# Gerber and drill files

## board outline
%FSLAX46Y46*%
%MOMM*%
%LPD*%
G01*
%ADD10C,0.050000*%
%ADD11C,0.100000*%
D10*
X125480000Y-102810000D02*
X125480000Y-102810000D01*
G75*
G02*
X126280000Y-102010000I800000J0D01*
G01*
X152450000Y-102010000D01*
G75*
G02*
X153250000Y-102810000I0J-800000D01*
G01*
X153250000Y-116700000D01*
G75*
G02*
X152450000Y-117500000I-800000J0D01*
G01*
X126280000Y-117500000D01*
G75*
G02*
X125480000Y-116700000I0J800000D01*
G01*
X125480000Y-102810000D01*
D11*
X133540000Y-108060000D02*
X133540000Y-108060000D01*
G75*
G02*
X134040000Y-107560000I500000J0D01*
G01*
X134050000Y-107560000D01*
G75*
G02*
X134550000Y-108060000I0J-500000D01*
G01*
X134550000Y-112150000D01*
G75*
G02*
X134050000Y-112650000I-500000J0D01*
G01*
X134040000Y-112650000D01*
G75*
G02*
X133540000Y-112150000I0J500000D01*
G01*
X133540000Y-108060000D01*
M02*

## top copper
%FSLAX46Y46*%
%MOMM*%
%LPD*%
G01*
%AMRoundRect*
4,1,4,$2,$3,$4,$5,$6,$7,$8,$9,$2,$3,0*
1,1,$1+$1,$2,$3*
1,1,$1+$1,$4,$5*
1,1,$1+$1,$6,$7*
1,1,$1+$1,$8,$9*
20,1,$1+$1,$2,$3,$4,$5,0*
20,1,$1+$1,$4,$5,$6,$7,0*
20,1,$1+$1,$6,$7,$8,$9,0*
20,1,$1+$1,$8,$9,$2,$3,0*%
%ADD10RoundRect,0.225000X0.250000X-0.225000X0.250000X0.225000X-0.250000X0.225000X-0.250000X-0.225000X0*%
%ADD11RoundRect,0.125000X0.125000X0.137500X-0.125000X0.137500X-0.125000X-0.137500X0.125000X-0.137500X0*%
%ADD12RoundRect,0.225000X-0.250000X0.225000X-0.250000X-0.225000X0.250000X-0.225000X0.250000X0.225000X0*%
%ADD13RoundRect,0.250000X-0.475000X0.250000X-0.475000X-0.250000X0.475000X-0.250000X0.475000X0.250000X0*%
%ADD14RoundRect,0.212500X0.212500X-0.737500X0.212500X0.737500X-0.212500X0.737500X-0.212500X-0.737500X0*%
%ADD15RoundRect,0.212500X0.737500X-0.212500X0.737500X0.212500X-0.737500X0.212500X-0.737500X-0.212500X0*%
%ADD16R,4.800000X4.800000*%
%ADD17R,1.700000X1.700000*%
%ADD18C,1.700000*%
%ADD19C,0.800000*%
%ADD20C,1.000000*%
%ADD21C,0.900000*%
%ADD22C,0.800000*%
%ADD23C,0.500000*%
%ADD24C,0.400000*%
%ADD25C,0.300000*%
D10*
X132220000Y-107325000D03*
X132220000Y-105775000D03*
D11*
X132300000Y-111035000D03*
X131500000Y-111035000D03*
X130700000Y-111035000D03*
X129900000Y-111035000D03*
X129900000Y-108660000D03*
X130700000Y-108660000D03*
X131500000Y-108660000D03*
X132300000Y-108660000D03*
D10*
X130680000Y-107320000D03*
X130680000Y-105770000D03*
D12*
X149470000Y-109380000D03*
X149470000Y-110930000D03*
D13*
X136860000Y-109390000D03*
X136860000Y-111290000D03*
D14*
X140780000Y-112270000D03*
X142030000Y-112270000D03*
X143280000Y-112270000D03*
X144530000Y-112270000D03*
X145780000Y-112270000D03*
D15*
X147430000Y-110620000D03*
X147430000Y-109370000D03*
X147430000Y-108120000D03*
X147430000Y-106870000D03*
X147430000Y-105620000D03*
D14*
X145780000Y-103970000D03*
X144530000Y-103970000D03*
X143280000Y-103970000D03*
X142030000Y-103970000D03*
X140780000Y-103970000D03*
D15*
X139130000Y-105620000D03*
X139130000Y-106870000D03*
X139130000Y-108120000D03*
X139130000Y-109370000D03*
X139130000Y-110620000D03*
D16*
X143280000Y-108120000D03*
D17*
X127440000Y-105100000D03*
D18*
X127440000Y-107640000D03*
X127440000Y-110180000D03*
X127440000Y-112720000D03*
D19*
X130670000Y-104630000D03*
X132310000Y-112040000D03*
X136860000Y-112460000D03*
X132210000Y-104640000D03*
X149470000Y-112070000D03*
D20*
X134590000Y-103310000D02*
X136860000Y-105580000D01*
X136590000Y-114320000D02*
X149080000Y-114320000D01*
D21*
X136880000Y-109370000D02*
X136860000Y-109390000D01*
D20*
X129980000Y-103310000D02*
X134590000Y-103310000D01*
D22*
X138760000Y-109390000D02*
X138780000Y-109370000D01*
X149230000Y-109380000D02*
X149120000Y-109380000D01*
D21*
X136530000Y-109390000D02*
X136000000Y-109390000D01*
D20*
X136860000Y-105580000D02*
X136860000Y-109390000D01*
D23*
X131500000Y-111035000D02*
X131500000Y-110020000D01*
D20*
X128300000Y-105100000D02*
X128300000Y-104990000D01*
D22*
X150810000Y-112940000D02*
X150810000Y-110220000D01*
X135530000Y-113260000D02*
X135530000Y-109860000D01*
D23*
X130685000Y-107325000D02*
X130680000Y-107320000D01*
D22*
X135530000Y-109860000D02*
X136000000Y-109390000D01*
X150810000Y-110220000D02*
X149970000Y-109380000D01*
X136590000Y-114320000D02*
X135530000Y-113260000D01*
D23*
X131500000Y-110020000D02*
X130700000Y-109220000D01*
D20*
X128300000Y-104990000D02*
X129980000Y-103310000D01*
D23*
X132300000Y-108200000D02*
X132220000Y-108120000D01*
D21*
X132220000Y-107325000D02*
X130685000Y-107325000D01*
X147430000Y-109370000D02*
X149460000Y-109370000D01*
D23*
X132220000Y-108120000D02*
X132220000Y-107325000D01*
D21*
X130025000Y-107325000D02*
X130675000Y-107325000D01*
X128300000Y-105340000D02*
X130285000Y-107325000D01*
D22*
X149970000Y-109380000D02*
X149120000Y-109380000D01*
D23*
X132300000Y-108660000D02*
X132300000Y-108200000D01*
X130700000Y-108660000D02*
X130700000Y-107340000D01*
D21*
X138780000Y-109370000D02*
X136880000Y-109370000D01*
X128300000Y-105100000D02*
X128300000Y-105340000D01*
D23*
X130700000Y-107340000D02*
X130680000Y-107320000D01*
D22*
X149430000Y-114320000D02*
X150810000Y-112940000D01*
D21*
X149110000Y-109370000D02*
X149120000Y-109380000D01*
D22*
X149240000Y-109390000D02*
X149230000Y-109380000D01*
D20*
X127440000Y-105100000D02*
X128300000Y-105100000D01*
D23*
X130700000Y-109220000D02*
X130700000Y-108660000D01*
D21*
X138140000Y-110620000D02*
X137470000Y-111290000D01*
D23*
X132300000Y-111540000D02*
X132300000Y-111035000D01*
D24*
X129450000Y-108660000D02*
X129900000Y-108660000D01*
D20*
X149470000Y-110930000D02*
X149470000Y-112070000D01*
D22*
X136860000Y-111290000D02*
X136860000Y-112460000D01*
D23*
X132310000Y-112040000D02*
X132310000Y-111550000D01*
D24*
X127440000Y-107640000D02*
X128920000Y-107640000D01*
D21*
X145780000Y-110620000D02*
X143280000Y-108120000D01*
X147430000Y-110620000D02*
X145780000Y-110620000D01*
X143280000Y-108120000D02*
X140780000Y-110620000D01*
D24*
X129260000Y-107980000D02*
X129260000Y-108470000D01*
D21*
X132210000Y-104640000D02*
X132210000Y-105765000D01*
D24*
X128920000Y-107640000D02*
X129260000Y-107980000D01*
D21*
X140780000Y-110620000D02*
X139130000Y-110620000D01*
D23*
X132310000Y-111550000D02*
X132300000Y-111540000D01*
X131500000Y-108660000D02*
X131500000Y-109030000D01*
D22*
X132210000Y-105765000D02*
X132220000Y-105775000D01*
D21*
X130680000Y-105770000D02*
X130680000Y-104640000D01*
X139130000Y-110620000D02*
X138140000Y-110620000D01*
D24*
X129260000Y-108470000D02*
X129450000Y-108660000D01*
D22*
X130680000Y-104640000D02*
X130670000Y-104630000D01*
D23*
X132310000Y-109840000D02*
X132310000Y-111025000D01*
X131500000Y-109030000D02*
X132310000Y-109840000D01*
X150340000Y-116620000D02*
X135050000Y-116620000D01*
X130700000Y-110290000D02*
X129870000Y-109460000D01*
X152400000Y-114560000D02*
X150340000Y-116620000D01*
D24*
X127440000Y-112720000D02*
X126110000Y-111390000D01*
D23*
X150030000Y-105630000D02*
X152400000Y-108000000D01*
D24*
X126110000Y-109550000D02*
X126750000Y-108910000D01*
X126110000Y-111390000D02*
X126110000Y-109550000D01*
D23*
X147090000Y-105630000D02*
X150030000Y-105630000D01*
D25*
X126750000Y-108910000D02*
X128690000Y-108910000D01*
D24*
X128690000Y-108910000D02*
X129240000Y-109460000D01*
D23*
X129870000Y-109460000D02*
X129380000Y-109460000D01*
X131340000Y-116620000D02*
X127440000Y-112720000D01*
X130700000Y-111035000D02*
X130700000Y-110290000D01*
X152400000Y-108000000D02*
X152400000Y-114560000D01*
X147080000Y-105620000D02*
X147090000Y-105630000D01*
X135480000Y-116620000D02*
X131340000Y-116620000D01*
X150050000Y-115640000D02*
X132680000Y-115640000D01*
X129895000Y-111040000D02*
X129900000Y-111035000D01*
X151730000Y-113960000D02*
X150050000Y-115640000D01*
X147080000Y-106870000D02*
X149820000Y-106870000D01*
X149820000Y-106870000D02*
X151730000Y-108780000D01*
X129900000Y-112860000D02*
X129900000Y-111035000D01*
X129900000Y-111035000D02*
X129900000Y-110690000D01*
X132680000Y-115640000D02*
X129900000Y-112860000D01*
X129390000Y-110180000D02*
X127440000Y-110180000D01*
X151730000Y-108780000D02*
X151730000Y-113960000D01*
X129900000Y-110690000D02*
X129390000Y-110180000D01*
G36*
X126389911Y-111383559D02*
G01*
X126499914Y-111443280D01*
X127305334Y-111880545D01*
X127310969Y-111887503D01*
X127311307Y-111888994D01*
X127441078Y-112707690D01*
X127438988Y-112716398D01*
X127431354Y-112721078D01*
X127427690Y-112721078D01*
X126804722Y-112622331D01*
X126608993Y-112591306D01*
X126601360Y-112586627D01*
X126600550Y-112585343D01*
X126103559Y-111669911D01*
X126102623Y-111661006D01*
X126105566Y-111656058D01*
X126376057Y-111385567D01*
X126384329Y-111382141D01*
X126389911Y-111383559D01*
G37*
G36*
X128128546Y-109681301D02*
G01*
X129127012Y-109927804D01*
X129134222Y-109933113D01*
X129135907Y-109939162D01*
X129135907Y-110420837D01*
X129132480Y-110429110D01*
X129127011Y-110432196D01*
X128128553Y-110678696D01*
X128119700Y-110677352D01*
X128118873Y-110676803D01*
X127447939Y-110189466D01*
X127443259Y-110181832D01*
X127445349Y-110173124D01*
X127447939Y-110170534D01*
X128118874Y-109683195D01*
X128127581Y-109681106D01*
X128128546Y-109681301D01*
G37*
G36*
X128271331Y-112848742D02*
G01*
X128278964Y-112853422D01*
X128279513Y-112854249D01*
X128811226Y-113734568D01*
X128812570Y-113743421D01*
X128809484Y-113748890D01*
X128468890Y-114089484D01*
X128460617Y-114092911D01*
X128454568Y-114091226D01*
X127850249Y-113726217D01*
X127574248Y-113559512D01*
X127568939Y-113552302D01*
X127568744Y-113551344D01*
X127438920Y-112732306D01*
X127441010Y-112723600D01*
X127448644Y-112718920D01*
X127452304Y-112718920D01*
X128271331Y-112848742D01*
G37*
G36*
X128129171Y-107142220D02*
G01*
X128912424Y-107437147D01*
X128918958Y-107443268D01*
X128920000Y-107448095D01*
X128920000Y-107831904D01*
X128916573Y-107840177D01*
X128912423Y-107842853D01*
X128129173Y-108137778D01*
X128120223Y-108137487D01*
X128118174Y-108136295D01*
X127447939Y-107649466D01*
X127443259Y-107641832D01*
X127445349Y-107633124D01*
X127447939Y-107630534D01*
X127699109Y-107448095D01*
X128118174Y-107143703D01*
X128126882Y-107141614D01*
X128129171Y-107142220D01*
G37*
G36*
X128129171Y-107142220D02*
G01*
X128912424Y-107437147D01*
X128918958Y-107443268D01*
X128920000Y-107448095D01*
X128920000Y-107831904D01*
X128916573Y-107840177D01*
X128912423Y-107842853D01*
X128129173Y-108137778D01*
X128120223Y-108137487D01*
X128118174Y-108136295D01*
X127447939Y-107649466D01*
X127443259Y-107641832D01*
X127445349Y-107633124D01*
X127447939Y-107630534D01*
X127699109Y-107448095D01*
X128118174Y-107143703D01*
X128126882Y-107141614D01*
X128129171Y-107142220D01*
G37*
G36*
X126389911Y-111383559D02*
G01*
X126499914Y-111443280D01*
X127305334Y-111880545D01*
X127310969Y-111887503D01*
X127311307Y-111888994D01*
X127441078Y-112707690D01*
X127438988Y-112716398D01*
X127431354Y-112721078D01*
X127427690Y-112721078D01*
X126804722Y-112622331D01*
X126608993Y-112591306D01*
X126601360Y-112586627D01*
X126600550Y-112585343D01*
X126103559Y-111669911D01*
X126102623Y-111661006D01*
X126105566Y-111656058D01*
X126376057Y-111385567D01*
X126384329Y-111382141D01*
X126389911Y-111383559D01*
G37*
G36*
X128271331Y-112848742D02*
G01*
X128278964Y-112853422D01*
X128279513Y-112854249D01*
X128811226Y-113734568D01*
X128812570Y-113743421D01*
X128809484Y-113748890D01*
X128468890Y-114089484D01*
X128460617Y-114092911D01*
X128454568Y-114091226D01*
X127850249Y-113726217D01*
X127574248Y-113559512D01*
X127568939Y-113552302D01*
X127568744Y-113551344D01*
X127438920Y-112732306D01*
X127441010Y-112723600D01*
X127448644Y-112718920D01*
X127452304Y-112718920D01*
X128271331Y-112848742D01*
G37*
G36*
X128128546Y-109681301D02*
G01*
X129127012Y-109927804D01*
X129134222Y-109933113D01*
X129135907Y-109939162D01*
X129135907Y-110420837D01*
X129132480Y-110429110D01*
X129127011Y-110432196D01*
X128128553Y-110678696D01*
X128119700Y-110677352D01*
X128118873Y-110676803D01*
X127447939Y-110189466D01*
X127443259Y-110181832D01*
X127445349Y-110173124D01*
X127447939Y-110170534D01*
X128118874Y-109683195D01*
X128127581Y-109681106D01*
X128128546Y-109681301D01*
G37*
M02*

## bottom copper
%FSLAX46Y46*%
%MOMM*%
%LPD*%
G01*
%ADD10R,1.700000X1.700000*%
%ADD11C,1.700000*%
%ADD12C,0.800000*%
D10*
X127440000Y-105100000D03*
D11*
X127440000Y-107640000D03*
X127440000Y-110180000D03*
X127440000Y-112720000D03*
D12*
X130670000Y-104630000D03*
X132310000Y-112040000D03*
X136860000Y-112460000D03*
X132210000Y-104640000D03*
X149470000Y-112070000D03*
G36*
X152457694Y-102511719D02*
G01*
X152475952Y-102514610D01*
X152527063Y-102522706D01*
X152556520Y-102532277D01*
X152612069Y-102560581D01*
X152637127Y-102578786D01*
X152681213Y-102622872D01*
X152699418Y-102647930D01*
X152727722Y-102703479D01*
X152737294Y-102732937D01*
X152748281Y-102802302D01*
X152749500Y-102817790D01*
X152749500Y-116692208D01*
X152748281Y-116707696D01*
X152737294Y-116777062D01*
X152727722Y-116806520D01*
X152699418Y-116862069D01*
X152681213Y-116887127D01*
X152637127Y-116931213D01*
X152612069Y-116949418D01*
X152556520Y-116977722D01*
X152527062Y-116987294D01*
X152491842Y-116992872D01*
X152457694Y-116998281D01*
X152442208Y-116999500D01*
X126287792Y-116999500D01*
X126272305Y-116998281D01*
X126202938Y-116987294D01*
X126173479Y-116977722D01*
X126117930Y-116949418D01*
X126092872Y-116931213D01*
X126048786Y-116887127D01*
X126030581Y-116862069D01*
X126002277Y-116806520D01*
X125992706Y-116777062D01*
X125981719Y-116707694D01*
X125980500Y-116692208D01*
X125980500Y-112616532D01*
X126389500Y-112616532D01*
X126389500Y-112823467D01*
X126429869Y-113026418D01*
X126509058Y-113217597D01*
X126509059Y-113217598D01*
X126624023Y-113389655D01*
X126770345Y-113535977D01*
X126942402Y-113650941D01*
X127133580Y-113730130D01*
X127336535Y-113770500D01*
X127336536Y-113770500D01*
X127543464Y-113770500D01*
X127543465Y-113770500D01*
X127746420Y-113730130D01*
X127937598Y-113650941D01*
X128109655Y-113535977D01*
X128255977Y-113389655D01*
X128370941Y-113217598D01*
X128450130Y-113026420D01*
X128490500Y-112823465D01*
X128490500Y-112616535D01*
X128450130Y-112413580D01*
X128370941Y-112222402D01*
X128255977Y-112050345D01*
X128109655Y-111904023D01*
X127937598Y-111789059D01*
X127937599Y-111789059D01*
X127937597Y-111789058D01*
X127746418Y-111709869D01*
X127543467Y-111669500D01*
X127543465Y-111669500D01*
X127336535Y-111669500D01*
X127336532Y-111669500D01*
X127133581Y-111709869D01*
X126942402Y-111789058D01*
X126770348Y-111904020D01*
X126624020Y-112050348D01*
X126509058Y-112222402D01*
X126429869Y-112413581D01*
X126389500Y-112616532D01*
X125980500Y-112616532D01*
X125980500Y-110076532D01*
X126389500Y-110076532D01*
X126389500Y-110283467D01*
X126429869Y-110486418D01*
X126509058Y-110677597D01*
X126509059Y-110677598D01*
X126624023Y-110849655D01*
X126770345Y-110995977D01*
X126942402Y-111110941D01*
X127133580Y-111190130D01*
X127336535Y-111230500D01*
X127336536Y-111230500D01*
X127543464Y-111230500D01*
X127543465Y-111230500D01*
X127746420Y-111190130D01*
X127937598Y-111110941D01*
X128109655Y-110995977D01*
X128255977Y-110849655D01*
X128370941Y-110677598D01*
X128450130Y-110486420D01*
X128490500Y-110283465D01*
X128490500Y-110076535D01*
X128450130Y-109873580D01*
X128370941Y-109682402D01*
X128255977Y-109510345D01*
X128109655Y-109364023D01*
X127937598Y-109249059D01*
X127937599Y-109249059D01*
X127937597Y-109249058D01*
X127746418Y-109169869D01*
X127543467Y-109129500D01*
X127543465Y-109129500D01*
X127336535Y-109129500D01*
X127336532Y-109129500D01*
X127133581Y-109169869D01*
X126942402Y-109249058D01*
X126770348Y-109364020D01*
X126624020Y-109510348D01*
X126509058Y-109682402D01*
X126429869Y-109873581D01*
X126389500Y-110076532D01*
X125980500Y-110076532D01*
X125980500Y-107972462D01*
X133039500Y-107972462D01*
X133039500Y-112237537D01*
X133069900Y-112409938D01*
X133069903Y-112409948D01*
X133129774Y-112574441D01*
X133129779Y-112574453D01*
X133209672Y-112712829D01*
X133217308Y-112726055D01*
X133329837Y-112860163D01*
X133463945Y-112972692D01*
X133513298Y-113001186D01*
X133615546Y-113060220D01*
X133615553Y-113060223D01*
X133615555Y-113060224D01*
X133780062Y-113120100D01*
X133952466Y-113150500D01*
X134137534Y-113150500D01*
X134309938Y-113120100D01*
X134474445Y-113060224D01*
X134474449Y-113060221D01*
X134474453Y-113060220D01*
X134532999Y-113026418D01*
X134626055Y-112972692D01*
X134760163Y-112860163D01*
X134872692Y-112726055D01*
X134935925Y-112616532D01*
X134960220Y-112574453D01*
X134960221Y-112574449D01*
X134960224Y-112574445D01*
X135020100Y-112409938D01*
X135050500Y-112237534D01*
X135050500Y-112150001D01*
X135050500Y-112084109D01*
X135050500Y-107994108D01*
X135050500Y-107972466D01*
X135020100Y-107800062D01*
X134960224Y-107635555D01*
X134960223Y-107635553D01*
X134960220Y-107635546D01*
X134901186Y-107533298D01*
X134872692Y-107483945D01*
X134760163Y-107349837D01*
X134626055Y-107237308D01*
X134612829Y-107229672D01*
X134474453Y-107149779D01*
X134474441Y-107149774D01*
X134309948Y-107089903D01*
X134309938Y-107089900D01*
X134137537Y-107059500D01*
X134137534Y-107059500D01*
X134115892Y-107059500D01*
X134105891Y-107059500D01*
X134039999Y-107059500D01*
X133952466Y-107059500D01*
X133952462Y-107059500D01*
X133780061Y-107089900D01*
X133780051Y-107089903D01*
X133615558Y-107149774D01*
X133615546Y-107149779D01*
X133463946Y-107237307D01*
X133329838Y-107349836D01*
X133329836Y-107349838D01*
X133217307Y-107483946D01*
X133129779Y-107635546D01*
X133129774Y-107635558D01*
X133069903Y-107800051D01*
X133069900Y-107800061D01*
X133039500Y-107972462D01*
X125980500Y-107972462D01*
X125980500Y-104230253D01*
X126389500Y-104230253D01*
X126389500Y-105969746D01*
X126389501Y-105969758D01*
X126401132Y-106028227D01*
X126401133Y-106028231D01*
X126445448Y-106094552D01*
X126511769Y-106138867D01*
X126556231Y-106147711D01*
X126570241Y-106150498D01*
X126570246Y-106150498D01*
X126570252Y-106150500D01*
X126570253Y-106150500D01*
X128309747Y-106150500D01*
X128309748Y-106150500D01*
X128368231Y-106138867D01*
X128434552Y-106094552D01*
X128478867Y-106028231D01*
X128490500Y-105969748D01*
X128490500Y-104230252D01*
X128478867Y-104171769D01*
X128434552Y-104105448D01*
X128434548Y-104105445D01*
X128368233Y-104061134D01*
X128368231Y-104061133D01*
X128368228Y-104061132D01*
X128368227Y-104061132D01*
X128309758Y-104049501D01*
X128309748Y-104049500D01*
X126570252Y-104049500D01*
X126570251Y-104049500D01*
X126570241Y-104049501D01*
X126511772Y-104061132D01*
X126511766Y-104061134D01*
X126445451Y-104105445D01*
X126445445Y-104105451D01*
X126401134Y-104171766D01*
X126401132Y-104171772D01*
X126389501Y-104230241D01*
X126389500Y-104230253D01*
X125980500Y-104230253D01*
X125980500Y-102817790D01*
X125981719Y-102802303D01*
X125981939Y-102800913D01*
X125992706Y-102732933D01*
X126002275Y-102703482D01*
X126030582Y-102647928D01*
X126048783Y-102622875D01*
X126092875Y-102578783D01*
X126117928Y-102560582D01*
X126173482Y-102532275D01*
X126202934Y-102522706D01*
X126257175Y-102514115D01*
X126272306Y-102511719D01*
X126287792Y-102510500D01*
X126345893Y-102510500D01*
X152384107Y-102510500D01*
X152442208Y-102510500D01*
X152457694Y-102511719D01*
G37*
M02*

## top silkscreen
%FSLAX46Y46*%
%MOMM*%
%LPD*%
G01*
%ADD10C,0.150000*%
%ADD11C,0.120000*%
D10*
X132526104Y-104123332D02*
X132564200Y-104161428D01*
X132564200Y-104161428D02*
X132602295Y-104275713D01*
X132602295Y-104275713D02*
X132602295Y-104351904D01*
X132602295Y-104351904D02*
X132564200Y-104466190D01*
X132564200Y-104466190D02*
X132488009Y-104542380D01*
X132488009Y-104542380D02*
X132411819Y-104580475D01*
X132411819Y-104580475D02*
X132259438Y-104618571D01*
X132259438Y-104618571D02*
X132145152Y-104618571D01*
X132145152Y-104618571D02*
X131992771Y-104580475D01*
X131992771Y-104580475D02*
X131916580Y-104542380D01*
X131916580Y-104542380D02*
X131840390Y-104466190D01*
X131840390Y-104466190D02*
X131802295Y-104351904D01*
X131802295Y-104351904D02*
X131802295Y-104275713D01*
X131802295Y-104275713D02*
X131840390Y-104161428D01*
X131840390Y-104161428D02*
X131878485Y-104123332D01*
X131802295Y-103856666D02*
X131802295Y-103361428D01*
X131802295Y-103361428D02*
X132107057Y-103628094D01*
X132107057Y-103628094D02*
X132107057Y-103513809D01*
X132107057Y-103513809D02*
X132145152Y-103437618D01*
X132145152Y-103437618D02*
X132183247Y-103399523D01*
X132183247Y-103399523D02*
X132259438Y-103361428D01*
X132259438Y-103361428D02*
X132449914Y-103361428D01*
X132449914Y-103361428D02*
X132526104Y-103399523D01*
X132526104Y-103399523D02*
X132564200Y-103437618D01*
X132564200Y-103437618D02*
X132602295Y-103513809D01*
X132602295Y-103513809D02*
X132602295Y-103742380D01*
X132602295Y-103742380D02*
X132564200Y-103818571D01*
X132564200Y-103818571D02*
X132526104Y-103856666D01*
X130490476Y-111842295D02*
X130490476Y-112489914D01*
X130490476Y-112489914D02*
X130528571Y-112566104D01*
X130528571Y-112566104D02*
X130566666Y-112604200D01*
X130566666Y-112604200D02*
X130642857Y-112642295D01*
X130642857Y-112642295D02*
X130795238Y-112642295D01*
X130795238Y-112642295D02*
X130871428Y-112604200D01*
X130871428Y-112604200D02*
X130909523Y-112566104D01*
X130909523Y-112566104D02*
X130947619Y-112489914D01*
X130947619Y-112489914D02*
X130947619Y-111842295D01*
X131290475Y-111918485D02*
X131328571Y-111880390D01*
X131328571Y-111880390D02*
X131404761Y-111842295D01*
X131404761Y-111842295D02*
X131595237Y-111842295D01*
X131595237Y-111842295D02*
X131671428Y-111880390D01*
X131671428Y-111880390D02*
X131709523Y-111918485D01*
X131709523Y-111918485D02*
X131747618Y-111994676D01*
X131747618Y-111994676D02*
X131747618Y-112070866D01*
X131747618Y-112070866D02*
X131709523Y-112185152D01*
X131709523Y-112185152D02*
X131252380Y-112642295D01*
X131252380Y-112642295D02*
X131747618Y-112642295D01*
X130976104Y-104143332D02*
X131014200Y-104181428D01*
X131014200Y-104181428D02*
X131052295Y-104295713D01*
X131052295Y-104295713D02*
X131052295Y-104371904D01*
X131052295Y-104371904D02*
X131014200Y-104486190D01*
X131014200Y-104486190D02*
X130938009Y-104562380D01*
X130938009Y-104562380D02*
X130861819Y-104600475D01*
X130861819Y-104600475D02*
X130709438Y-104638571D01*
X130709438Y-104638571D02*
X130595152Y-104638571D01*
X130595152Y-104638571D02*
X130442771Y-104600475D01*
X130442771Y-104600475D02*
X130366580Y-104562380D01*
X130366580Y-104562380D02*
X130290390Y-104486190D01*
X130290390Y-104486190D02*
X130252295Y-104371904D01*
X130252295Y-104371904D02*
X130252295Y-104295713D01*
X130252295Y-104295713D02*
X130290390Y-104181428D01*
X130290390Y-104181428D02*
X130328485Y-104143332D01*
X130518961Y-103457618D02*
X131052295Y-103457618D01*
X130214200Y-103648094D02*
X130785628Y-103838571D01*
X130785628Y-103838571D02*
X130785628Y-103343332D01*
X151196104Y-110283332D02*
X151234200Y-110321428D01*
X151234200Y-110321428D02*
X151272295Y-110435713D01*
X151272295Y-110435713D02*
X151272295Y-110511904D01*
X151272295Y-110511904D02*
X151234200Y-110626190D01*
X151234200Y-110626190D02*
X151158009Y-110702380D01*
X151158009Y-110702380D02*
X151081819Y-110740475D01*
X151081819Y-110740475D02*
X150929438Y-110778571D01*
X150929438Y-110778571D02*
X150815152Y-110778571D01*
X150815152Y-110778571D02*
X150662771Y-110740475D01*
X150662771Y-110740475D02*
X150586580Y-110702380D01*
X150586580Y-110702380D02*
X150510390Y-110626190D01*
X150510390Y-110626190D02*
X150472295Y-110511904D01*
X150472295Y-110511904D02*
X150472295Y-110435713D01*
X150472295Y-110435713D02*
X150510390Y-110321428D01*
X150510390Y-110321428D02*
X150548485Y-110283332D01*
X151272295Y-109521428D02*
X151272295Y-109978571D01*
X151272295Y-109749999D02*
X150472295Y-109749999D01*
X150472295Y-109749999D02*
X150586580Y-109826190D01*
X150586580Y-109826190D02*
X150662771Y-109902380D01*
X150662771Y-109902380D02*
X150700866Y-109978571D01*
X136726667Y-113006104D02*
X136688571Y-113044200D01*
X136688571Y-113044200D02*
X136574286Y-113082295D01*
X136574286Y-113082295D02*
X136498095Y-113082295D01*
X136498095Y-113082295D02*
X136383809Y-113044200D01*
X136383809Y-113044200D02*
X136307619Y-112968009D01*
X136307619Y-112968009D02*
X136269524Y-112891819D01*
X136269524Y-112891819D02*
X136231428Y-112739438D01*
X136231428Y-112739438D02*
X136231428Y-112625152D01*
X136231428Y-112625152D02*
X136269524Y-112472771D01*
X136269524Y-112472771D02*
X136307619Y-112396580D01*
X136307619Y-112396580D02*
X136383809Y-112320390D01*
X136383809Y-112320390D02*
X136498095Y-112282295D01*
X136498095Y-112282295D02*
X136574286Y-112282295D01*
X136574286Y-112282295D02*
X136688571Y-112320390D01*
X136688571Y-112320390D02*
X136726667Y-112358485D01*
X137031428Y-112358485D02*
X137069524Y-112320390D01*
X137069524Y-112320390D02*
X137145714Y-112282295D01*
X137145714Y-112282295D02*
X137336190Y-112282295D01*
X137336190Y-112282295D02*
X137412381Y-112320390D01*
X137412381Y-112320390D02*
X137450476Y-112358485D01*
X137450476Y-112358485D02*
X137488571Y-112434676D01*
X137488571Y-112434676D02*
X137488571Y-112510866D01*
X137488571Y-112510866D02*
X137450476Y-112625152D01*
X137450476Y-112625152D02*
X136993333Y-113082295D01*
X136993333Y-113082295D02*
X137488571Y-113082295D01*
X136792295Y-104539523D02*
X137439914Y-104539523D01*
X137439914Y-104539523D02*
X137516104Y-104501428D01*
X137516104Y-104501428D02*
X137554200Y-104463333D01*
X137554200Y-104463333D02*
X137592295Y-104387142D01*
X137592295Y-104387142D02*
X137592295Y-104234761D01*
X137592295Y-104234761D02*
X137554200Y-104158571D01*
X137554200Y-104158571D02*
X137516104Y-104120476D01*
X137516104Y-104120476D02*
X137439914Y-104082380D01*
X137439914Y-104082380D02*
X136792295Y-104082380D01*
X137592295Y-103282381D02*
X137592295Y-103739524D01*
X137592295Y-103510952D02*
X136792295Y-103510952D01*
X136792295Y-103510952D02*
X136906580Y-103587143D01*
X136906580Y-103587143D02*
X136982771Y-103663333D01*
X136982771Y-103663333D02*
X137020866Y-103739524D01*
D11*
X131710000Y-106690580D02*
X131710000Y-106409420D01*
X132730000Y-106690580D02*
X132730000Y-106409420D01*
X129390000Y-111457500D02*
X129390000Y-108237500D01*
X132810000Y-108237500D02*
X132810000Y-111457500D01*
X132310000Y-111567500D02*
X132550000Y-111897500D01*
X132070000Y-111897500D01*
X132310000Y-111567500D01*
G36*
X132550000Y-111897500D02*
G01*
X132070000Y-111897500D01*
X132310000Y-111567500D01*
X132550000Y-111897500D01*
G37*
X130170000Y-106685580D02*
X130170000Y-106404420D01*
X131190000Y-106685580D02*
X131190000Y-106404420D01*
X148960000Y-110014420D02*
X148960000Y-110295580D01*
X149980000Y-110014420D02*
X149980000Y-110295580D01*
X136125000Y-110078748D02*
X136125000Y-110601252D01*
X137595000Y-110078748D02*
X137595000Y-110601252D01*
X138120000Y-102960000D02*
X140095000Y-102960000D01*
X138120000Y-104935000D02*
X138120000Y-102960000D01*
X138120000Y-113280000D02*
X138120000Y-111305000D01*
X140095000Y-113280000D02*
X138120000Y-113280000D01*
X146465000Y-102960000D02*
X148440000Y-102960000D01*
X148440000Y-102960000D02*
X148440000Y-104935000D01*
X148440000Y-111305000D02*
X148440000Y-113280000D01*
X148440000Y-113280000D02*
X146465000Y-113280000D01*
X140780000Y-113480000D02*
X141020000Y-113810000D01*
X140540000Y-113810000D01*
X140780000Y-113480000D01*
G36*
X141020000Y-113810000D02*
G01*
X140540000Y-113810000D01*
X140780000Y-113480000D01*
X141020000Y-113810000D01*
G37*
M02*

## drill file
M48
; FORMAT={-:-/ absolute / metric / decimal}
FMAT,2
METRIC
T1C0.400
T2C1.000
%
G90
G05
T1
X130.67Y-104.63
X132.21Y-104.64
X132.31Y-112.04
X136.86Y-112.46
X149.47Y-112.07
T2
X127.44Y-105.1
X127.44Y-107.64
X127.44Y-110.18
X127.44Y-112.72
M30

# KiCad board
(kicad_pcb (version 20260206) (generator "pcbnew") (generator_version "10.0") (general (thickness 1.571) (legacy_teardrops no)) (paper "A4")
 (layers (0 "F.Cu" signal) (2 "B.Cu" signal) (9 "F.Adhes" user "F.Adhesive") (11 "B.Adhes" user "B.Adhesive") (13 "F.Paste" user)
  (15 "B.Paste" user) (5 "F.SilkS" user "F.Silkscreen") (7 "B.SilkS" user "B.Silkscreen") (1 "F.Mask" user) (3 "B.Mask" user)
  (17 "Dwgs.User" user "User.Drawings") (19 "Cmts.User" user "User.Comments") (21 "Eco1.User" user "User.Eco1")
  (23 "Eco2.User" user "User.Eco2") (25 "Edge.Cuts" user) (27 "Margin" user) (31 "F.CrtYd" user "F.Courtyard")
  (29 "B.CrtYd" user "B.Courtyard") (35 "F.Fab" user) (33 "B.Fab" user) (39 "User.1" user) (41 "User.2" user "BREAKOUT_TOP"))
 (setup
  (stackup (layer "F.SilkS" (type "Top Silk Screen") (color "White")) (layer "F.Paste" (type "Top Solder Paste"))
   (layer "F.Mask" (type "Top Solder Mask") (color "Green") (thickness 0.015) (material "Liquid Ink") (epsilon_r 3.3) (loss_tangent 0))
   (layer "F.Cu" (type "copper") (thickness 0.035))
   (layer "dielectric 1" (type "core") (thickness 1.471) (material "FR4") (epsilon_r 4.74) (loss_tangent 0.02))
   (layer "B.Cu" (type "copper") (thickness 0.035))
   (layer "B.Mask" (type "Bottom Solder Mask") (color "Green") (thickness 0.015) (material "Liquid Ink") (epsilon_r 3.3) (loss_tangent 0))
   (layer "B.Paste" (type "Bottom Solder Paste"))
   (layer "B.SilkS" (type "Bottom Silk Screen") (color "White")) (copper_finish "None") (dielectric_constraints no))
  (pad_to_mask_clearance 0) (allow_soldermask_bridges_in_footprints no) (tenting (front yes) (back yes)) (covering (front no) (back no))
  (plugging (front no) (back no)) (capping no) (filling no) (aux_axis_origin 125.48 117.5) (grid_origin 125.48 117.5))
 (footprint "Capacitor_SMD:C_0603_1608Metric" (layer "F.Cu") (at 132.22 106.55 90)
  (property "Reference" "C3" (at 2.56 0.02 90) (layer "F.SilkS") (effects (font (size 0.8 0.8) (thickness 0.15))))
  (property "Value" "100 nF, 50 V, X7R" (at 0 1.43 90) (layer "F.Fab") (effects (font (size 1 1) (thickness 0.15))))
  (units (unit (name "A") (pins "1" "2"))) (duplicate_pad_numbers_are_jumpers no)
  (fp_line (start -0.14058 -0.51) (end 0.14058 -0.51) (stroke (width 0.12) (type solid)) (layer "F.SilkS"))
  (fp_line (start -0.14058 0.51) (end 0.14058 0.51) (stroke (width 0.12) (type solid)) (layer "F.SilkS"))
  (pad "1" smd roundrect (at -0.775 0 90) (size 0.9 0.95) (layers "F.Cu" "F.Mask" "F.Paste") (roundrect_rratio 0.25) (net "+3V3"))
  (pad "2" smd roundrect (at 0.775 0 90) (size 0.9 0.95) (layers "F.Cu" "F.Mask" "F.Paste") (roundrect_rratio 0.25) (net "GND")))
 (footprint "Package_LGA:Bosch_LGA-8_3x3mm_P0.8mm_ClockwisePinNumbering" (layer "F.Cu") (at 131.1 109.8475 180)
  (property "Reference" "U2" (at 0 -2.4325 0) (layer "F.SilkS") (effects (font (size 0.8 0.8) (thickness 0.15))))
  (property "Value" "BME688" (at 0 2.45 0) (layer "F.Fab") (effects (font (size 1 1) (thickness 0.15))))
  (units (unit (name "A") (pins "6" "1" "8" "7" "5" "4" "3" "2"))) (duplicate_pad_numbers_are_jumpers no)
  (fp_line (start 1.71 -1.61) (end 1.71 1.61) (stroke (width 0.12) (type solid)) (layer "F.SilkS"))
  (fp_line (start -1.71 1.61) (end -1.71 -1.61) (stroke (width 0.12) (type solid)) (layer "F.SilkS"))
  (fp_poly (pts (xy -1.21 -1.72) (xy -1.45 -2.05) (xy -0.97 -2.05)) (stroke (width 0.12) (type solid)) (fill yes) (layer "F.SilkS"))
  (pad "1" smd roundrect (at -1.2 -1.1875 180) (size 0.5 0.525) (layers "F.Cu" "F.Mask" "F.Paste") (roundrect_rratio 0.25) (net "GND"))
  (pad "2" smd roundrect (at -0.4 -1.1875 180) (size 0.5 0.525) (layers "F.Cu" "F.Mask" "F.Paste") (roundrect_rratio 0.25) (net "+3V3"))
  (pad "3" smd roundrect (at 0.4 -1.1875 180) (size 0.5 0.525) (layers "F.Cu" "F.Mask" "F.Paste") (roundrect_rratio 0.25) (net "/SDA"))
  (pad "4" smd roundrect (at 1.2 -1.1875 180) (size 0.5 0.525) (layers "F.Cu" "F.Mask" "F.Paste") (roundrect_rratio 0.25) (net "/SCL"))
  (pad "5" smd roundrect (at 1.2 1.1875 180) (size 0.5 0.525) (layers "F.Cu" "F.Mask" "F.Paste") (roundrect_rratio 0.25) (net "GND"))
  (pad "6" smd roundrect (at 0.4 1.1875 180) (size 0.5 0.525) (layers "F.Cu" "F.Mask" "F.Paste") (roundrect_rratio 0.25) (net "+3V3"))
  (pad "7" smd roundrect (at -0.4 1.1875 180) (size 0.5 0.525) (layers "F.Cu" "F.Mask" "F.Paste") (roundrect_rratio 0.25) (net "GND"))
  (pad "8" smd roundrect (at -1.2 1.1875 180) (size 0.5 0.525) (layers "F.Cu" "F.Mask" "F.Paste") (roundrect_rratio 0.25) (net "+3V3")))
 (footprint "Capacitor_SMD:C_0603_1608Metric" (layer "F.Cu") (at 130.68 106.545 90)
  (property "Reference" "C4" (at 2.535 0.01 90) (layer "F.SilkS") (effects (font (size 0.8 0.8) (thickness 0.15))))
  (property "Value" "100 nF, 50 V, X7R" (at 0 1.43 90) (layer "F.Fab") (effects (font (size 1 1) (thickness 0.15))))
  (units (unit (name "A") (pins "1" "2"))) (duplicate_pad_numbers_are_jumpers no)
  (fp_line (start -0.14058 -0.51) (end 0.14058 -0.51) (stroke (width 0.12) (type solid)) (layer "F.SilkS"))
  (fp_line (start -0.14058 0.51) (end 0.14058 0.51) (stroke (width 0.12) (type solid)) (layer "F.SilkS"))
  (pad "1" smd roundrect (at -0.775 0 90) (size 0.9 0.95) (layers "F.Cu" "F.Mask" "F.Paste") (roundrect_rratio 0.25) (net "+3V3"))
  (pad "2" smd roundrect (at 0.775 0 90) (size 0.9 0.95) (layers "F.Cu" "F.Mask" "F.Paste") (roundrect_rratio 0.25) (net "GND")))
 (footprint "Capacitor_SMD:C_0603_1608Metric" (layer "F.Cu") (at 149.47 110.155 -90)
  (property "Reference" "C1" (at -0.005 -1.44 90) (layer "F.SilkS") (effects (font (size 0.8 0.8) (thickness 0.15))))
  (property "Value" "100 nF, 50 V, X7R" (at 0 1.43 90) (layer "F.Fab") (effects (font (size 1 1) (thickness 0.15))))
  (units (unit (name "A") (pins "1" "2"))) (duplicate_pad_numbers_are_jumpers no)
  (fp_line (start -0.14058 0.51) (end 0.14058 0.51) (stroke (width 0.12) (type solid)) (layer "F.SilkS"))
  (fp_line (start -0.14058 -0.51) (end 0.14058 -0.51) (stroke (width 0.12) (type solid)) (layer "F.SilkS"))
  (pad "1" smd roundrect (at -0.775 0 270) (size 0.9 0.95) (layers "F.Cu" "F.Mask" "F.Paste") (roundrect_rratio 0.25) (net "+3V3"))
  (pad "2" smd roundrect (at 0.775 0 270) (size 0.9 0.95) (layers "F.Cu" "F.Mask" "F.Paste") (roundrect_rratio 0.25) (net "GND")))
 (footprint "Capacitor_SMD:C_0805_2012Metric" (layer "F.Cu") (at 136.86 110.34 -90)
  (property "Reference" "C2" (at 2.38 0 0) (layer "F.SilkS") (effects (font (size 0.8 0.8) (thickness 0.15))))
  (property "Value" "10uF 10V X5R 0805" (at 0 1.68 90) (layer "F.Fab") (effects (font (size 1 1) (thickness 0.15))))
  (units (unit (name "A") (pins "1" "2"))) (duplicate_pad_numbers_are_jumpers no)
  (fp_line (start -0.261252 0.735) (end 0.261252 0.735) (stroke (width 0.12) (type solid)) (layer "F.SilkS"))
  (fp_line (start -0.261252 -0.735) (end 0.261252 -0.735) (stroke (width 0.12) (type solid)) (layer "F.SilkS"))
  (pad "1" smd roundrect (at -0.95 0 270) (size 1 1.45) (layers "F.Cu" "F.Mask" "F.Paste") (roundrect_rratio 0.25) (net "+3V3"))
  (pad "2" smd roundrect (at 0.95 0 270) (size 1 1.45) (layers "F.Cu" "F.Mask" "F.Paste") (roundrect_rratio 0.25) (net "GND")))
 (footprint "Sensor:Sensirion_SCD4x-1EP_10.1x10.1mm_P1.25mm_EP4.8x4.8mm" (layer "F.Cu") (at 143.28 108.12 90)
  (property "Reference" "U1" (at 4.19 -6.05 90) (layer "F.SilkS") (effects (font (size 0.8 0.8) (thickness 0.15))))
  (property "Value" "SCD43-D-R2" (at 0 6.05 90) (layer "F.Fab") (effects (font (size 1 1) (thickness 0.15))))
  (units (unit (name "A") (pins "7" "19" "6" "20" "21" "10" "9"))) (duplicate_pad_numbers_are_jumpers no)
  (fp_line (start 5.16 -5.16) (end 5.16 -3.185) (stroke (width 0.12) (type solid)) (layer "F.SilkS"))
  (fp_line (start 3.185 -5.16) (end 5.16 -5.16) (stroke (width 0.12) (type solid)) (layer "F.SilkS"))
  (fp_line (start -5.16 -5.16) (end -3.185 -5.16) (stroke (width 0.12) (type solid)) (layer "F.SilkS"))
  (fp_line (start -5.16 -3.185) (end -5.16 -5.16) (stroke (width 0.12) (type solid)) (layer "F.SilkS"))
  (fp_line (start 5.16 3.185) (end 5.16 5.16) (stroke (width 0.12) (type solid)) (layer "F.SilkS"))
  (fp_line (start 5.16 5.16) (end 3.185 5.16) (stroke (width 0.12) (type solid)) (layer "F.SilkS"))
  (fp_line (start -3.185 5.16) (end -5.16 5.16) (stroke (width 0.12) (type solid)) (layer "F.SilkS"))
  (fp_line (start -5.16 5.16) (end -5.16 3.185) (stroke (width 0.12) (type solid)) (layer "F.SilkS"))
  (fp_poly (pts (xy -5.36 -2.5) (xy -5.69 -2.26) (xy -5.69 -2.74)) (stroke (width 0.12) (type solid)) (fill yes) (layer "F.SilkS"))
  (pad "" smd roundrect (at -1.2 -1.2 90) (size 1.93 1.93) (layers "F.Paste") (roundrect_rratio 0.129534))
  (pad "" smd roundrect (at -1.2 1.2 90) (size 1.93 1.93) (layers "F.Paste") (roundrect_rratio 0.129534))
  (pad "" smd roundrect (at 1.2 -1.2 90) (size 1.93 1.93) (layers "F.Paste") (roundrect_rratio 0.129534))
  (pad "" smd roundrect (at 1.2 1.2 90) (size 1.93 1.93) (layers "F.Paste") (roundrect_rratio 0.129534))
  (pad "1" smd roundrect (at -4.15 -2.5 90) (size 1.9 0.85) (layers "F.Cu" "F.Mask" "F.Paste") (roundrect_rratio 0.25))
  (pad "2" smd roundrect (at -4.15 -1.25 90) (size 1.9 0.85) (layers "F.Cu" "F.Mask" "F.Paste") (roundrect_rratio 0.25))
  (pad "3" smd roundrect (at -4.15 0 90) (size 1.9 0.85) (layers "F.Cu" "F.Mask" "F.Paste") (roundrect_rratio 0.25))
  (pad "4" smd roundrect (at -4.15 1.25 90) (size 1.9 0.85) (layers "F.Cu" "F.Mask" "F.Paste") (roundrect_rratio 0.25))
  (pad "5" smd roundrect (at -4.15 2.5 90) (size 1.9 0.85) (layers "F.Cu" "F.Mask" "F.Paste") (roundrect_rratio 0.25))
  (pad "6" smd roundrect (at -2.5 4.15 90) (size 0.85 1.9) (layers "F.Cu" "F.Mask" "F.Paste") (roundrect_rratio 0.25) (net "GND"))
  (pad "7" smd roundrect (at -1.25 4.15 90) (size 0.85 1.9) (layers "F.Cu" "F.Mask" "F.Paste") (roundrect_rratio 0.25) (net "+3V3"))
  (pad "8" smd roundrect (at 0 4.15 90) (size 0.85 1.9) (layers "F.Cu" "F.Mask" "F.Paste") (roundrect_rratio 0.25))
  (pad "9" smd roundrect (at 1.25 4.15 90) (size 0.85 1.9) (layers "F.Cu" "F.Mask" "F.Paste") (roundrect_rratio 0.25) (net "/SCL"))
  (pad "10" smd roundrect (at 2.5 4.15 90) (size 0.85 1.9) (layers "F.Cu" "F.Mask" "F.Paste") (roundrect_rratio 0.25) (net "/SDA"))
  (pad "11" smd roundrect (at 4.15 2.5 90) (size 1.9 0.85) (layers "F.Cu" "F.Mask" "F.Paste") (roundrect_rratio 0.25))
  (pad "12" smd roundrect (at 4.15 1.25 90) (size 1.9 0.85) (layers "F.Cu" "F.Mask" "F.Paste") (roundrect_rratio 0.25))
  (pad "13" smd roundrect (at 4.15 0 90) (size 1.9 0.85) (layers "F.Cu" "F.Mask" "F.Paste") (roundrect_rratio 0.25))
  (pad "14" smd roundrect (at 4.15 -1.25 90) (size 1.9 0.85) (layers "F.Cu" "F.Mask" "F.Paste") (roundrect_rratio 0.25))
  (pad "15" smd roundrect (at 4.15 -2.5 90) (size 1.9 0.85) (layers "F.Cu" "F.Mask" "F.Paste") (roundrect_rratio 0.25))
  (pad "16" smd roundrect (at 2.5 -4.15 90) (size 0.85 1.9) (layers "F.Cu" "F.Mask" "F.Paste") (roundrect_rratio 0.25))
  (pad "17" smd roundrect (at 1.25 -4.15 90) (size 0.85 1.9) (layers "F.Cu" "F.Mask" "F.Paste") (roundrect_rratio 0.25))
  (pad "18" smd roundrect (at 0 -4.15 90) (size 0.85 1.9) (layers "F.Cu" "F.Mask" "F.Paste") (roundrect_rratio 0.25))
  (pad "19" smd roundrect (at -1.25 -4.15 90) (size 0.85 1.9) (layers "F.Cu" "F.Mask" "F.Paste") (roundrect_rratio 0.25) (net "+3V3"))
  (pad "20" smd roundrect (at -2.5 -4.15 90) (size 0.85 1.9) (layers "F.Cu" "F.Mask" "F.Paste") (roundrect_rratio 0.25) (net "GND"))
  (pad "21" smd rect (at 0 0 90) (size 4.8 4.8) (layers "F.Cu" "F.Mask") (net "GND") (zone_connect 2)))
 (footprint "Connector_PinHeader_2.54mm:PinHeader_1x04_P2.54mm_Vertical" (layer "B.Cu") (at 127.44 105.1 180)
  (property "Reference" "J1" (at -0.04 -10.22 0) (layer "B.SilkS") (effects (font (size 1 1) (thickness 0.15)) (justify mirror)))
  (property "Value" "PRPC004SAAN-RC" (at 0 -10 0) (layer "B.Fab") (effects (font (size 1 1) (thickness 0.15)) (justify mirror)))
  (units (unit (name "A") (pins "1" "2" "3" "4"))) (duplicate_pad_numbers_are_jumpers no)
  (pad "1" thru_hole rect (at 0 0 180) (size 1.7 1.7) (drill 1) (layers "*.Cu" "*.Mask") (remove_unused_layers no) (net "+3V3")
   (teardrops (best_length_ratio 0.5) (max_length 1) (best_width_ratio 1) (max_width 1) (curved_edges no) (filter_ratio 0.9) (enabled yes)
    (allow_two_segments no) (prefer_zone_connections yes)))
  (pad "2" thru_hole circle (at 0 -2.54 180) (size 1.7 1.7) (drill 1) (layers "*.Cu" "*.Mask") (remove_unused_layers no) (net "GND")
   (teardrops (best_length_ratio 0.5) (max_length 1) (best_width_ratio 1) (max_width 1) (curved_edges no) (filter_ratio 0.9) (enabled yes)
    (allow_two_segments no) (prefer_zone_connections yes)))
  (pad "3" thru_hole circle (at 0 -5.08 180) (size 1.7 1.7) (drill 1) (layers "*.Cu" "*.Mask") (remove_unused_layers no) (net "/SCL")
   (teardrops (best_length_ratio 0.5) (max_length 1) (best_width_ratio 1) (max_width 1) (curved_edges no) (filter_ratio 0.9) (enabled yes)
    (allow_two_segments no) (prefer_zone_connections yes)))
  (pad "4" thru_hole circle (at 0 -7.62 180) (size 1.7 1.7) (drill 1) (layers "*.Cu" "*.Mask") (remove_unused_layers no) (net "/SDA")
   (teardrops (best_length_ratio 0.5) (max_length 1) (best_width_ratio 1) (max_width 1) (curved_edges no) (filter_ratio 0.9) (enabled yes)
    (allow_two_segments no) (prefer_zone_connections yes))))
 (gr_rect (start 125.48 102.01) (end 153.25 117.5) (radius 0.8) (stroke (width 0.05) (type solid)) (fill no) (layer "Edge.Cuts"))
 (gr_rect (start 133.54 107.56) (end 134.55 112.65) (radius 0.5) (stroke (width 0.1) (type solid)) (fill no) (layer "Edge.Cuts"))
 (segment (start 134.59 103.31) (end 136.86 105.58) (width 1) (layer "F.Cu") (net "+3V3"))
 (segment (start 136.59 114.32) (end 149.08 114.32) (width 1) (layer "F.Cu") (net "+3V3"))
 (segment (start 136.88 109.37) (end 136.86 109.39) (width 0.9) (layer "F.Cu") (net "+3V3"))
 (segment (start 129.98 103.31) (end 134.59 103.31) (width 1) (layer "F.Cu") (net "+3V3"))
 (segment (start 138.76 109.39) (end 138.78 109.37) (width 0.8) (layer "F.Cu") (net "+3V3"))
 (segment (start 149.23 109.38) (end 149.12 109.38) (width 0.8) (layer "F.Cu") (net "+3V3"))
 (segment (start 136.53 109.39) (end 136 109.39) (width 0.9) (layer "F.Cu") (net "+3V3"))
 (segment (start 136.86 105.58) (end 136.86 109.39) (width 1) (layer "F.Cu") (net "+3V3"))
 (segment (start 131.5 111.035) (end 131.5 110.02) (width 0.5) (layer "F.Cu") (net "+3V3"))
 (segment (start 128.3 105.1) (end 128.3 104.99) (width 1) (layer "F.Cu") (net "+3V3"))
 (segment (start 150.81 112.94) (end 150.81 110.22) (width 0.8) (layer "F.Cu") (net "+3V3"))
 (segment (start 135.53 113.26) (end 135.53 109.86) (width 0.8) (layer "F.Cu") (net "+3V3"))
 (segment (start 130.685 107.325) (end 130.68 107.32) (width 0.5) (layer "F.Cu") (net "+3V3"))
 (segment (start 135.53 109.86) (end 136 109.39) (width 0.8) (layer "F.Cu") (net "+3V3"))
 (segment (start 150.81 110.22) (end 149.97 109.38) (width 0.8) (layer "F.Cu") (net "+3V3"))
 (segment (start 136.59 114.32) (end 135.53 113.26) (width 0.8) (layer "F.Cu") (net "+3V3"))
 (segment (start 131.5 110.02) (end 130.7 109.22) (width 0.5) (layer "F.Cu") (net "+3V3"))
 (segment (start 128.3 104.99) (end 129.98 103.31) (width 1) (layer "F.Cu") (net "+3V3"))
 (segment (start 132.3 108.2) (end 132.22 108.12) (width 0.5) (layer "F.Cu") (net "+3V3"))
 (segment (start 132.22 107.325) (end 130.685 107.325) (width 0.9) (layer "F.Cu") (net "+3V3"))
 (segment (start 147.43 109.37) (end 149.46 109.37) (width 0.9) (layer "F.Cu") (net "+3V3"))
 (segment (start 132.22 108.12) (end 132.22 107.325) (width 0.5) (layer "F.Cu") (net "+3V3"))
 (segment (start 130.025 107.325) (end 130.675 107.325) (width 0.9) (layer "F.Cu") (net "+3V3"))
 (segment (start 128.3 105.34) (end 130.285 107.325) (width 0.9) (layer "F.Cu") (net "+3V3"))
 (segment (start 149.97 109.38) (end 149.12 109.38) (width 0.8) (layer "F.Cu") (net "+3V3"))
 (segment (start 132.3 108.66) (end 132.3 108.2) (width 0.5) (layer "F.Cu") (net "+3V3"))
 (segment (start 130.7 108.66) (end 130.7 107.34) (width 0.5) (layer "F.Cu") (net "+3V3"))
 (segment (start 138.78 109.37) (end 136.88 109.37) (width 0.9) (layer "F.Cu") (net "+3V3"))
 (segment (start 128.3 105.1) (end 128.3 105.34) (width 0.9) (layer "F.Cu") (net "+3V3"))
 (segment (start 130.7 107.34) (end 130.68 107.32) (width 0.5) (layer "F.Cu") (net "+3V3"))
 (segment (start 149.43 114.32) (end 150.81 112.94) (width 0.8) (layer "F.Cu") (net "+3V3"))
 (segment (start 149.11 109.37) (end 149.12 109.38) (width 0.9) (layer "F.Cu") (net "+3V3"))
 (segment (start 149.24 109.39) (end 149.23 109.38) (width 0.8) (layer "F.Cu") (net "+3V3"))
 (segment (start 127.44 105.1) (end 128.3 105.1) (width 1) (layer "F.Cu") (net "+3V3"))
 (segment (start 130.7 109.22) (end 130.7 108.66) (width 0.5) (layer "F.Cu") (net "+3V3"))
 (segment (start 138.14 110.62) (end 137.47 111.29) (width 0.9) (layer "F.Cu") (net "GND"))
 (segment (start 132.3 111.54) (end 132.3 111.035) (width 0.5) (layer "F.Cu") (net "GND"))
 (segment (start 129.45 108.66) (end 129.9 108.66) (width 0.4) (layer "F.Cu") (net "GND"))
 (segment (start 149.47 110.93) (end 149.47 112.07) (width 1) (layer "F.Cu") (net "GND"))
 (segment (start 136.86 111.29) (end 136.86 112.46) (width 0.8) (layer "F.Cu") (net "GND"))
 (segment (start 132.31 112.04) (end 132.31 111.55) (width 0.5) (layer "F.Cu") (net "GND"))
 (segment (start 127.44 107.64) (end 128.92 107.64) (width 0.4) (layer "F.Cu") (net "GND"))
 (segment (start 145.78 110.62) (end 143.28 108.12) (width 0.9) (layer "F.Cu") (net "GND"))
 (segment (start 147.43 110.62) (end 145.78 110.62) (width 0.9) (layer "F.Cu") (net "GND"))
 (segment (start 143.28 108.12) (end 140.78 110.62) (width 0.9) (layer "F.Cu") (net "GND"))
 (segment (start 129.26 107.98) (end 129.26 108.47) (width 0.4) (layer "F.Cu") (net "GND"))
 (segment (start 132.21 104.64) (end 132.21 105.765) (width 0.9) (layer "F.Cu") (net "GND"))
 (segment (start 128.92 107.64) (end 129.26 107.98) (width 0.4) (layer "F.Cu") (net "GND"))
 (segment (start 140.78 110.62) (end 139.13 110.62) (width 0.9) (layer "F.Cu") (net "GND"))
 (segment (start 132.31 111.55) (end 132.3 111.54) (width 0.5) (layer "F.Cu") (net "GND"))
 (segment (start 131.5 108.66) (end 131.5 109.03) (width 0.5) (layer "F.Cu") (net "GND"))
 (segment (start 132.21 105.765) (end 132.22 105.775) (width 0.8) (layer "F.Cu") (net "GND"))
 (segment (start 130.68 105.77) (end 130.68 104.64) (width 0.9) (layer "F.Cu") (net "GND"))
 (segment (start 139.13 110.62) (end 138.14 110.62) (width 0.9) (layer "F.Cu") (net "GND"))
 (segment (start 129.26 108.47) (end 129.45 108.66) (width 0.4) (layer "F.Cu") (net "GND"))
 (segment (start 130.68 104.64) (end 130.67 104.63) (width 0.8) (layer "F.Cu") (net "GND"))
 (segment (start 132.31 109.84) (end 132.31 111.025) (width 0.5) (layer "F.Cu") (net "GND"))
 (segment (start 131.5 109.03) (end 132.31 109.84) (width 0.5) (layer "F.Cu") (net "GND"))
 (via (at 130.67 104.63) (size 0.8) (drill 0.4) (layers "F.Cu" "B.Cu") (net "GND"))
 (via (at 132.31 112.04) (size 0.8) (drill 0.4) (layers "F.Cu" "B.Cu") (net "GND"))
 (via (at 136.86 112.46) (size 0.8) (drill 0.4) (layers "F.Cu" "B.Cu") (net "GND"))
 (via (at 132.21 104.64) (size 0.8) (drill 0.4) (layers "F.Cu" "B.Cu") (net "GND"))
 (via (at 149.47 112.07) (size 0.8) (drill 0.4) (layers "F.Cu" "B.Cu") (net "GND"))
 (segment (start 150.34 116.62) (end 135.05 116.62) (width 0.5) (layer "F.Cu") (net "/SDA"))
 (segment (start 130.7 110.29) (end 129.87 109.46) (width 0.5) (layer "F.Cu") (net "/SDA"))
 (segment (start 152.4 114.56) (end 150.34 116.62) (width 0.5) (layer "F.Cu") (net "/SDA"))
 (segment (start 127.44 112.72) (end 126.11 111.39) (width 0.4) (layer "F.Cu") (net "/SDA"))
 (segment (start 150.03 105.63) (end 152.4 108) (width 0.5) (layer "F.Cu") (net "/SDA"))
 (segment (start 126.11 109.55) (end 126.75 108.91) (width 0.4) (layer "F.Cu") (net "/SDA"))
 (segment (start 126.11 111.39) (end 126.11 109.55) (width 0.4) (layer "F.Cu") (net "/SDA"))
 (segment (start 147.09 105.63) (end 150.03 105.63) (width 0.5) (layer "F.Cu") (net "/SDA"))
 (segment (start 126.75 108.91) (end 128.69 108.91) (width 0.3) (layer "F.Cu") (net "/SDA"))
 (segment (start 128.69 108.91) (end 129.24 109.46) (width 0.4) (layer "F.Cu") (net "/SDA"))
 (segment (start 129.87 109.46) (end 129.38 109.46) (width 0.5) (layer "F.Cu") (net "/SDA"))
 (segment (start 131.34 116.62) (end 127.44 112.72) (width 0.5) (layer "F.Cu") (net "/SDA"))
 (segment (start 130.7 111.035) (end 130.7 110.29) (width 0.5) (layer "F.Cu") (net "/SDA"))
 (segment (start 152.4 108) (end 152.4 114.56) (width 0.5) (layer "F.Cu") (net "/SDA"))
 (segment (start 147.08 105.62) (end 147.09 105.63) (width 0.5) (layer "F.Cu") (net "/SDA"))
 (segment (start 135.48 116.62) (end 131.34 116.62) (width 0.5) (layer "F.Cu") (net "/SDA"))
 (segment (start 150.05 115.64) (end 132.68 115.64) (width 0.5) (layer "F.Cu") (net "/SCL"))
 (segment (start 129.895 111.04) (end 129.9 111.035) (width 0.5) (layer "F.Cu") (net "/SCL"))
 (segment (start 151.73 113.96) (end 150.05 115.64) (width 0.5) (layer "F.Cu") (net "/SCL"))
 (segment (start 147.08 106.87) (end 149.82 106.87) (width 0.5) (layer "F.Cu") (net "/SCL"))
 (segment (start 149.82 106.87) (end 151.73 108.78) (width 0.5) (layer "F.Cu") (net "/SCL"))
 (segment (start 129.9 112.86) (end 129.9 111.035) (width 0.5) (layer "F.Cu") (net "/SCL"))
 (segment (start 129.9 111.035) (end 129.9 110.69) (width 0.5) (layer "F.Cu") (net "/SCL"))
 (segment (start 132.68 115.64) (end 129.9 112.86) (width 0.5) (layer "F.Cu") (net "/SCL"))
 (segment (start 129.39 110.18) (end 127.44 110.18) (width 0.5) (layer "F.Cu") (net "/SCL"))
 (segment (start 151.73 108.78) (end 151.73 113.96) (width 0.5) (layer "F.Cu") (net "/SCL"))
 (segment (start 129.9 110.69) (end 129.39 110.18) (width 0.5) (layer "F.Cu") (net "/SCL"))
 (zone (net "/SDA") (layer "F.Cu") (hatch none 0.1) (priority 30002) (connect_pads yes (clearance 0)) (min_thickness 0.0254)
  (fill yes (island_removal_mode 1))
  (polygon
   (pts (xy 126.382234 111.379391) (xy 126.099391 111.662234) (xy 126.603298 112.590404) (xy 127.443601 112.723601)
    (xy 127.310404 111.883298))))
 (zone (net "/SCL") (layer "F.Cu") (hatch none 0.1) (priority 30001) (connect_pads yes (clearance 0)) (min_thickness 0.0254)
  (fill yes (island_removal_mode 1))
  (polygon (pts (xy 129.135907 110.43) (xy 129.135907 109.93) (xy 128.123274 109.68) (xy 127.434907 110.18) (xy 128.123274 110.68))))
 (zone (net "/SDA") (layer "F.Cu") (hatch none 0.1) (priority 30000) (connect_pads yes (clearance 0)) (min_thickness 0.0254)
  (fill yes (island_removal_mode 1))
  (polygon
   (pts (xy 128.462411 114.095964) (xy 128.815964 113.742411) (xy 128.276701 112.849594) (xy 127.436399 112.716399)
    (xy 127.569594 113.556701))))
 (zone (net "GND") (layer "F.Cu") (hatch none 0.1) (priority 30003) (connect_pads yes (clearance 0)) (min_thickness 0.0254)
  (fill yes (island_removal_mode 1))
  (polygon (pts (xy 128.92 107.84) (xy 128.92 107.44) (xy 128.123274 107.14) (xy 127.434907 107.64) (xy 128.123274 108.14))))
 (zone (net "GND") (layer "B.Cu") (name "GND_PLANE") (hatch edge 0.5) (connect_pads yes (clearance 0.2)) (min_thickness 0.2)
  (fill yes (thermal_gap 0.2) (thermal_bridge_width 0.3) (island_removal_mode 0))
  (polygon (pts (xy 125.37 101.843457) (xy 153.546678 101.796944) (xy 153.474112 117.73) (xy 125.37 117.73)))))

